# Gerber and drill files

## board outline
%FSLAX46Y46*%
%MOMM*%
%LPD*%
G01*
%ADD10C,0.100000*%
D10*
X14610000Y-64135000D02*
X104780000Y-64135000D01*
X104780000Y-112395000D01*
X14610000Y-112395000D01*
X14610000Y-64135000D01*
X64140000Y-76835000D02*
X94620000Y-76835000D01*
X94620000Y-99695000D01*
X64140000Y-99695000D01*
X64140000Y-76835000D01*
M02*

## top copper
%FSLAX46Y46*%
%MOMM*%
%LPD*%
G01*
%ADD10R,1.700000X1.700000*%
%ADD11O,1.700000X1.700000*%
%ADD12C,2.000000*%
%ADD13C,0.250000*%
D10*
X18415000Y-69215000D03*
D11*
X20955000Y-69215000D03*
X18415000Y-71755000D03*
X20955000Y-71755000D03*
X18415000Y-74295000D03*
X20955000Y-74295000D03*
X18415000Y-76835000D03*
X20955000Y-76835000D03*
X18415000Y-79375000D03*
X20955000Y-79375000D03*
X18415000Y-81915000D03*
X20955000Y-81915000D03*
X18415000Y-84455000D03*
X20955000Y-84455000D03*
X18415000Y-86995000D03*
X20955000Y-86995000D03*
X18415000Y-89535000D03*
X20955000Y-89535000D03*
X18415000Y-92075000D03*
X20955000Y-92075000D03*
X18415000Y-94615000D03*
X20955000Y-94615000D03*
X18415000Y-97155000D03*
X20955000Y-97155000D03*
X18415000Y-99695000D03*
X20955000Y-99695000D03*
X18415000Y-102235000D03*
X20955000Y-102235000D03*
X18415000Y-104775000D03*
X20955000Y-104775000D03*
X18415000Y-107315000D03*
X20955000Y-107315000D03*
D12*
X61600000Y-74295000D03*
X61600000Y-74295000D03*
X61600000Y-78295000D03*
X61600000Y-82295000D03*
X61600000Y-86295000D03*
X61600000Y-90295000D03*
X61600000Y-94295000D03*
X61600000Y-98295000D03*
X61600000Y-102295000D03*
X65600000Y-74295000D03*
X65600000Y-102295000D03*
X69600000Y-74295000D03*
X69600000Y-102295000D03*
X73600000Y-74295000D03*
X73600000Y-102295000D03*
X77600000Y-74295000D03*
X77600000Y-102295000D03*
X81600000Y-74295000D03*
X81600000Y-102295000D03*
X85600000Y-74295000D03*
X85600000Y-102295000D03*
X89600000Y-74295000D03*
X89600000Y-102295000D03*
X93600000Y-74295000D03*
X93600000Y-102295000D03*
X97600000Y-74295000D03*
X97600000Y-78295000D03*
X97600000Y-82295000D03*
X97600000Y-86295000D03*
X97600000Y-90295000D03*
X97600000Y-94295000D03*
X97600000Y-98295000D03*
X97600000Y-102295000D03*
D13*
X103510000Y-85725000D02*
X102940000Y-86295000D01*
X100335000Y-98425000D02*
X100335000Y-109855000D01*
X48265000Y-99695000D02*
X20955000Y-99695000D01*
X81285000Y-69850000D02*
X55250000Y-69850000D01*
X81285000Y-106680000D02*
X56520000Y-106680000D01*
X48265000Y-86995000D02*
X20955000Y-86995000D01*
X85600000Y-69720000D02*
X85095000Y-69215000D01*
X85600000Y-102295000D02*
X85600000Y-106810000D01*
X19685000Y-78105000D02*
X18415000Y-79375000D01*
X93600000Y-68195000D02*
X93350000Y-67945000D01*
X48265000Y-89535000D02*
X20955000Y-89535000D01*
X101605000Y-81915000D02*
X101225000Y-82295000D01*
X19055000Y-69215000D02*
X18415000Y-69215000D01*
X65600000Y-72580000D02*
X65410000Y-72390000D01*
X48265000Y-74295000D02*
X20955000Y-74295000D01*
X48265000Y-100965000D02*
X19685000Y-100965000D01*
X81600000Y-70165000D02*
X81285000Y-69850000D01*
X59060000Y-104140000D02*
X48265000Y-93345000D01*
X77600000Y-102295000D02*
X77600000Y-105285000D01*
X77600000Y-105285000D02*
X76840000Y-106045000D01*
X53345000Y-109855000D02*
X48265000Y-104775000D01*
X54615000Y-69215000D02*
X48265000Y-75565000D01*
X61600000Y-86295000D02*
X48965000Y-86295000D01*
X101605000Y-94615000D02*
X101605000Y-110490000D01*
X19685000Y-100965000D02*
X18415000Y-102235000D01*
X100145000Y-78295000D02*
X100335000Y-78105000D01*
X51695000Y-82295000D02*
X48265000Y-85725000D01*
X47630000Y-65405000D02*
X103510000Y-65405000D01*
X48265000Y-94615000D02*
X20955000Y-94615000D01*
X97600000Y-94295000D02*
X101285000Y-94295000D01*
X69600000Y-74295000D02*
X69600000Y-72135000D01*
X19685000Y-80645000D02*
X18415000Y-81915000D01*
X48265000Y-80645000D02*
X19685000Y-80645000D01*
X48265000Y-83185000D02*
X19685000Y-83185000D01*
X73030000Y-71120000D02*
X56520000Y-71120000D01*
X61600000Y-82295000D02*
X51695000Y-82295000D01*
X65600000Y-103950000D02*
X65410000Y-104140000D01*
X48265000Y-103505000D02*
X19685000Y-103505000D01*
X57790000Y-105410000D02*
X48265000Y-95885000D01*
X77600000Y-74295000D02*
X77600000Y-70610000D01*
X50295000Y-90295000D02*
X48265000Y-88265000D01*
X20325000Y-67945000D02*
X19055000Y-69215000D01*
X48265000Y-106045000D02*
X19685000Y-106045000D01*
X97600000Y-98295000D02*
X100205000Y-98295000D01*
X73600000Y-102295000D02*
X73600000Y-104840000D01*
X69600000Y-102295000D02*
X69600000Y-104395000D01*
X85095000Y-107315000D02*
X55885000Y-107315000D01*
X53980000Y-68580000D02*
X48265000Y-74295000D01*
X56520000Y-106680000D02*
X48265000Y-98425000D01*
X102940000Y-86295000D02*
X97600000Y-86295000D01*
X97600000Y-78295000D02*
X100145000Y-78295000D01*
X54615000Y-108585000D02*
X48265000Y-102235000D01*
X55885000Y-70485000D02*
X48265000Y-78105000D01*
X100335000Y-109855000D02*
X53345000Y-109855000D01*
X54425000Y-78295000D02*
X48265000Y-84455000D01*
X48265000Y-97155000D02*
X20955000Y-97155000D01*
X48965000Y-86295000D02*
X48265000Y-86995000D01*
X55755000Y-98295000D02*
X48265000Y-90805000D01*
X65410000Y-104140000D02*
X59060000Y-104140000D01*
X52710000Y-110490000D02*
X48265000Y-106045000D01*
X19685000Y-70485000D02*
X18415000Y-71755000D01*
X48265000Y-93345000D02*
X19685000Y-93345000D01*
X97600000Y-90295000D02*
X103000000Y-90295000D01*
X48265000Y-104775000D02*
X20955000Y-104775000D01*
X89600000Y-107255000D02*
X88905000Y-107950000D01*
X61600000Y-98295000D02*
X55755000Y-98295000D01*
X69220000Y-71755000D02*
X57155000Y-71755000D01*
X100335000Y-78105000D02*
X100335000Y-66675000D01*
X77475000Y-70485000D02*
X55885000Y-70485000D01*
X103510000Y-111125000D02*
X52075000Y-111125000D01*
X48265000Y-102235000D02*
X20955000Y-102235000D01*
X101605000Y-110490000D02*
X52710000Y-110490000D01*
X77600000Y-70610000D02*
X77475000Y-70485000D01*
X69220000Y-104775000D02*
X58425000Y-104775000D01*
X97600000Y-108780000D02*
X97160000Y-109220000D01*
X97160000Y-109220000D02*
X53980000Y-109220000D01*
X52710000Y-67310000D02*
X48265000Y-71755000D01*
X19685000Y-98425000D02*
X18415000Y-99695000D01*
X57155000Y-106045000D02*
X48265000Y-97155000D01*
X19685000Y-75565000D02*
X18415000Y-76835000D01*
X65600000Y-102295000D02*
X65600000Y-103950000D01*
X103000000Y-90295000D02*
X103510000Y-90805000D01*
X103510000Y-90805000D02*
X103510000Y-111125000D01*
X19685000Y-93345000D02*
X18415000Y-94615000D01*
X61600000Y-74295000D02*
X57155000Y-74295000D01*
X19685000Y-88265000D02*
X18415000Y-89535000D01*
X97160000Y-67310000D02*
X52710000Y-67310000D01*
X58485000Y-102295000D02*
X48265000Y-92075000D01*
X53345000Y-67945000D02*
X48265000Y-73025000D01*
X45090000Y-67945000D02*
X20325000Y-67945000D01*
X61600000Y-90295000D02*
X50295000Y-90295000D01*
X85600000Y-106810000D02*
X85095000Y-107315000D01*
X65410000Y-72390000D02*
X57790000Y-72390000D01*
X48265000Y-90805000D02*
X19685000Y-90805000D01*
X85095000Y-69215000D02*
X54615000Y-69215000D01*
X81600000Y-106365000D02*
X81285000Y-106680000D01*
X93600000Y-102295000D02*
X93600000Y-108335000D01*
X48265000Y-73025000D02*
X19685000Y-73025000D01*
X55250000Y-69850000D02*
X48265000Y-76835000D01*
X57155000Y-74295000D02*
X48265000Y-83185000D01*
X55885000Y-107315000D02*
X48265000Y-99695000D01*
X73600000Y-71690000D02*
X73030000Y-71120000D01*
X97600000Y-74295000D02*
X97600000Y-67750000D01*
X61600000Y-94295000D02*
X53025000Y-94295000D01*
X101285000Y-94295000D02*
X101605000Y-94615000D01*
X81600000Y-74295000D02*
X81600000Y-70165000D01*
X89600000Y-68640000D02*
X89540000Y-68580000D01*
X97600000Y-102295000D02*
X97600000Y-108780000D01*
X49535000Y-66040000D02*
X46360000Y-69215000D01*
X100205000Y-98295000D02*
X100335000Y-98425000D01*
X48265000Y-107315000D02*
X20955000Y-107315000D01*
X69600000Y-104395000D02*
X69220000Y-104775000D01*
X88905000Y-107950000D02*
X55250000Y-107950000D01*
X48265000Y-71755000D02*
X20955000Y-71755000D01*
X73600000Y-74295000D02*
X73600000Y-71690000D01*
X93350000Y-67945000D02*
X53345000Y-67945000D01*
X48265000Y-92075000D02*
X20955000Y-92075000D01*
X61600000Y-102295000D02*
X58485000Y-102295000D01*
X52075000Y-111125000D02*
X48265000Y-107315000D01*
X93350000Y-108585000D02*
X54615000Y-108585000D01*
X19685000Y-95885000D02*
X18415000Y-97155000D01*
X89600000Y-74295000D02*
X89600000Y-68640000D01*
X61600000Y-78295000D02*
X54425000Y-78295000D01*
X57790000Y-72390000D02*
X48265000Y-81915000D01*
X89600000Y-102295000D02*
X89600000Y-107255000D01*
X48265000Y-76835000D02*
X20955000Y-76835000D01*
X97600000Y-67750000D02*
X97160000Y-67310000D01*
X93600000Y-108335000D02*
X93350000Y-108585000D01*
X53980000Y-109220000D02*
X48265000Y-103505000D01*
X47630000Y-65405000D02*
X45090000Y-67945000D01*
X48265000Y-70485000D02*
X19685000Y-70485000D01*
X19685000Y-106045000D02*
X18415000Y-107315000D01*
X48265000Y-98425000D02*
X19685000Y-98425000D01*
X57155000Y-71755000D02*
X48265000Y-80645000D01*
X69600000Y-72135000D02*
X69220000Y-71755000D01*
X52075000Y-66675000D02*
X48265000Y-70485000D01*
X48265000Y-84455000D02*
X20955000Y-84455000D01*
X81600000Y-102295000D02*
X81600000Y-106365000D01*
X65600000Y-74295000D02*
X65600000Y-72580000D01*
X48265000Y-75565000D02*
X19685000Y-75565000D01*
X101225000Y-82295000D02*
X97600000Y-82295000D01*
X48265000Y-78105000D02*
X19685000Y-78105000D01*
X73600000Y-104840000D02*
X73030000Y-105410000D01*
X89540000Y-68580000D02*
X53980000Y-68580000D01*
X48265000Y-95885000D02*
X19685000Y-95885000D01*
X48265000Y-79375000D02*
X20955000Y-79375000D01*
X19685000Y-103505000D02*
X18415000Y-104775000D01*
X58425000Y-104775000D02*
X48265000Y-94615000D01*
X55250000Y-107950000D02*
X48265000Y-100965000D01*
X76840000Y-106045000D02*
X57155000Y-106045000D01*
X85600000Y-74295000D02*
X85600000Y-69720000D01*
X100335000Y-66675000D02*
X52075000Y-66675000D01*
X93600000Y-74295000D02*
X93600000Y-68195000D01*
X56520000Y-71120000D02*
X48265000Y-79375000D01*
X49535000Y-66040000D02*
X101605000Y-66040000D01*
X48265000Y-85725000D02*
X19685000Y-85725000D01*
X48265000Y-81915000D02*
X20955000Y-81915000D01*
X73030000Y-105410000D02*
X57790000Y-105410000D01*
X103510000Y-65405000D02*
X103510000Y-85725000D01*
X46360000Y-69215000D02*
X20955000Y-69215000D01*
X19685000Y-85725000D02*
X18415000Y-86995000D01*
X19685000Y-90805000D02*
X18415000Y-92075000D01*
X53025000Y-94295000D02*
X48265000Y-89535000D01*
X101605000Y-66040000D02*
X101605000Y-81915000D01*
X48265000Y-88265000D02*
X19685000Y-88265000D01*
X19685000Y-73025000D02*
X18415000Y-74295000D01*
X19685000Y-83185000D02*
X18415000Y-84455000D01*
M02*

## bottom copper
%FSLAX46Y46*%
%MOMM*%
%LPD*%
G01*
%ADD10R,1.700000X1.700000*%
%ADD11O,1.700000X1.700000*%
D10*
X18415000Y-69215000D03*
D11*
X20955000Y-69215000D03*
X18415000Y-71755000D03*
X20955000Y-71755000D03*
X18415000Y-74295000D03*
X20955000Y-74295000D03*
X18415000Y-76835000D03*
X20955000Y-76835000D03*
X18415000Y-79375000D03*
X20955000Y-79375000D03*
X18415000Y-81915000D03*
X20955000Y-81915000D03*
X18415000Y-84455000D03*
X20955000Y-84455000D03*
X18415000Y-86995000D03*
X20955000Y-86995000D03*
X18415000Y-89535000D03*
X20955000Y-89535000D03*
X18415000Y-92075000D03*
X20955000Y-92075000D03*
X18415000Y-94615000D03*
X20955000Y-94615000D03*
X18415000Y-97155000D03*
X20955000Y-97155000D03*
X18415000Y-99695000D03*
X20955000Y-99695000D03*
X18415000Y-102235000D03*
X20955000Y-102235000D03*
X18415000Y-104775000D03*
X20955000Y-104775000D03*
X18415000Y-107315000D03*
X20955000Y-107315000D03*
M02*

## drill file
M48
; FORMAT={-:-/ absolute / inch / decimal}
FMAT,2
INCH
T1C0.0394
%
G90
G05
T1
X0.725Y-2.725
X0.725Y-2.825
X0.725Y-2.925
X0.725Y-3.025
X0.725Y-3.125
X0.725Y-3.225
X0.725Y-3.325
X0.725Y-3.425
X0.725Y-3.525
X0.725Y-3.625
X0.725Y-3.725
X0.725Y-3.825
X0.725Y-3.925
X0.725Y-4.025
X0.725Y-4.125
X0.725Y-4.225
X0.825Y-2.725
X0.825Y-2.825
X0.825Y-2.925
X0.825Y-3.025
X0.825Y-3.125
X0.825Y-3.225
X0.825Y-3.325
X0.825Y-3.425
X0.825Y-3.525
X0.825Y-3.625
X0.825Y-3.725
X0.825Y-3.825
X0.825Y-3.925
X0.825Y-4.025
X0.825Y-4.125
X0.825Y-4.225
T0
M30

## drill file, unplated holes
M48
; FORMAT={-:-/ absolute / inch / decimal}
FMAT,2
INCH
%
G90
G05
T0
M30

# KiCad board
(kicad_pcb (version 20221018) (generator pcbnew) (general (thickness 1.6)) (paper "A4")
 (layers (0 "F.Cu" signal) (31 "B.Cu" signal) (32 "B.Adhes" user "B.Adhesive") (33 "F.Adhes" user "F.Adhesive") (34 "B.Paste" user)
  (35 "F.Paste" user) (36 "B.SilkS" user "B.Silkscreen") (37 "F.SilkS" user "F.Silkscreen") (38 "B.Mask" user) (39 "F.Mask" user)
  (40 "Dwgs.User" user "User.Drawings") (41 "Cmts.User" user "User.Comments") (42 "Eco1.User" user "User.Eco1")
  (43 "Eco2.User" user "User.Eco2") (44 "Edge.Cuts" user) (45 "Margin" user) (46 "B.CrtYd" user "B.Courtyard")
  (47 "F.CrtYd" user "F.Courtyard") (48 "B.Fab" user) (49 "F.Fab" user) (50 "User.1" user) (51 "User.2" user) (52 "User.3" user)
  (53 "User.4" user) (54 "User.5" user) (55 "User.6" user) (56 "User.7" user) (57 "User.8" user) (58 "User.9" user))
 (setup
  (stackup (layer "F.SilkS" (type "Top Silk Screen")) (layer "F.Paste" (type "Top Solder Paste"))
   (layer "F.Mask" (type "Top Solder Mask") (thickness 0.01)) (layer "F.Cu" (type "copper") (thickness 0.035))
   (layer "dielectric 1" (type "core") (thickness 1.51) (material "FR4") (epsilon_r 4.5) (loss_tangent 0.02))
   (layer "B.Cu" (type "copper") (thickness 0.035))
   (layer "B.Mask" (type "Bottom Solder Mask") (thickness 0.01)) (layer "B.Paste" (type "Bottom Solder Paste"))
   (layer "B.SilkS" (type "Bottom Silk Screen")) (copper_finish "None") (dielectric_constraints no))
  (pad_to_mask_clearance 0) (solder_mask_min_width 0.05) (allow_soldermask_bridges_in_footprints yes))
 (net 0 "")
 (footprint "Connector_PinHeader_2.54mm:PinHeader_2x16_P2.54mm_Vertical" (layer "F.Cu") (at 18.415 69.215)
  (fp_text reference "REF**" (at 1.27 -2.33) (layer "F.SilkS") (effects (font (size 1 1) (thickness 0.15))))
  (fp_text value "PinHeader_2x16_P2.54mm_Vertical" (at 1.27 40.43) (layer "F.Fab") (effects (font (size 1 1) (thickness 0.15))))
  (pad "1" thru_hole rect (at 0 0) (size 1.7 1.7) (drill 1) (layers "*.Cu" "*.Mask"))
  (pad "2" thru_hole oval (at 2.54 0) (size 1.7 1.7) (drill 1) (layers "*.Cu" "*.Mask"))
  (pad "3" thru_hole oval (at 0 2.54) (size 1.7 1.7) (drill 1) (layers "*.Cu" "*.Mask"))
  (pad "4" thru_hole oval (at 2.54 2.54) (size 1.7 1.7) (drill 1) (layers "*.Cu" "*.Mask"))
  (pad "5" thru_hole oval (at 0 5.08) (size 1.7 1.7) (drill 1) (layers "*.Cu" "*.Mask"))
  (pad "6" thru_hole oval (at 2.54 5.08) (size 1.7 1.7) (drill 1) (layers "*.Cu" "*.Mask"))
  (pad "7" thru_hole oval (at 0 7.62) (size 1.7 1.7) (drill 1) (layers "*.Cu" "*.Mask"))
  (pad "8" thru_hole oval (at 2.54 7.62) (size 1.7 1.7) (drill 1) (layers "*.Cu" "*.Mask"))
  (pad "9" thru_hole oval (at 0 10.16) (size 1.7 1.7) (drill 1) (layers "*.Cu" "*.Mask"))
  (pad "10" thru_hole oval (at 2.54 10.16) (size 1.7 1.7) (drill 1) (layers "*.Cu" "*.Mask"))
  (pad "11" thru_hole oval (at 0 12.7) (size 1.7 1.7) (drill 1) (layers "*.Cu" "*.Mask"))
  (pad "12" thru_hole oval (at 2.54 12.7) (size 1.7 1.7) (drill 1) (layers "*.Cu" "*.Mask"))
  (pad "13" thru_hole oval (at 0 15.24) (size 1.7 1.7) (drill 1) (layers "*.Cu" "*.Mask"))
  (pad "14" thru_hole oval (at 2.54 15.24) (size 1.7 1.7) (drill 1) (layers "*.Cu" "*.Mask"))
  (pad "15" thru_hole oval (at 0 17.78) (size 1.7 1.7) (drill 1) (layers "*.Cu" "*.Mask"))
  (pad "16" thru_hole oval (at 2.54 17.78) (size 1.7 1.7) (drill 1) (layers "*.Cu" "*.Mask"))
  (pad "17" thru_hole oval (at 0 20.32) (size 1.7 1.7) (drill 1) (layers "*.Cu" "*.Mask"))
  (pad "18" thru_hole oval (at 2.54 20.32) (size 1.7 1.7) (drill 1) (layers "*.Cu" "*.Mask"))
  (pad "19" thru_hole oval (at 0 22.86) (size 1.7 1.7) (drill 1) (layers "*.Cu" "*.Mask"))
  (pad "20" thru_hole oval (at 2.54 22.86) (size 1.7 1.7) (drill 1) (layers "*.Cu" "*.Mask"))
  (pad "21" thru_hole oval (at 0 25.4) (size 1.7 1.7) (drill 1) (layers "*.Cu" "*.Mask"))
  (pad "22" thru_hole oval (at 2.54 25.4) (size 1.7 1.7) (drill 1) (layers "*.Cu" "*.Mask"))
  (pad "23" thru_hole oval (at 0 27.94) (size 1.7 1.7) (drill 1) (layers "*.Cu" "*.Mask"))
  (pad "24" thru_hole oval (at 2.54 27.94) (size 1.7 1.7) (drill 1) (layers "*.Cu" "*.Mask"))
  (pad "25" thru_hole oval (at 0 30.48) (size 1.7 1.7) (drill 1) (layers "*.Cu" "*.Mask"))
  (pad "26" thru_hole oval (at 2.54 30.48) (size 1.7 1.7) (drill 1) (layers "*.Cu" "*.Mask"))
  (pad "27" thru_hole oval (at 0 33.02) (size 1.7 1.7) (drill 1) (layers "*.Cu" "*.Mask"))
  (pad "28" thru_hole oval (at 2.54 33.02) (size 1.7 1.7) (drill 1) (layers "*.Cu" "*.Mask"))
  (pad "29" thru_hole oval (at 0 35.56) (size 1.7 1.7) (drill 1) (layers "*.Cu" "*.Mask"))
  (pad "30" thru_hole oval (at 2.54 35.56) (size 1.7 1.7) (drill 1) (layers "*.Cu" "*.Mask"))
  (pad "31" thru_hole oval (at 0 38.1) (size 1.7 1.7) (drill 1) (layers "*.Cu" "*.Mask"))
  (pad "32" thru_hole oval (at 2.54 38.1) (size 1.7 1.7) (drill 1) (layers "*.Cu" "*.Mask")))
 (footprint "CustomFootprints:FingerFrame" (layer "F.Cu") (at 61.6 74.295)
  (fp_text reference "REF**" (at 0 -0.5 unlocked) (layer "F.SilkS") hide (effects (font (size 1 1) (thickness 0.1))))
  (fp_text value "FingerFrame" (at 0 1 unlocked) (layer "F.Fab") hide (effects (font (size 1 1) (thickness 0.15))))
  (pad "1" smd circle (at 0 0) (size 2 2) (layers "F.Cu" "F.Paste" "F.Mask"))
  (pad "1" smd circle (at 0 0) (size 2 2) (layers "F.Cu" "F.Paste" "F.Mask"))
  (pad "1" smd circle (at 0 4) (size 2 2) (layers "F.Cu" "F.Paste" "F.Mask"))
  (pad "1" smd circle (at 0 8) (size 2 2) (layers "F.Cu" "F.Paste" "F.Mask"))
  (pad "1" smd circle (at 0 12) (size 2 2) (layers "F.Cu" "F.Paste" "F.Mask"))
  (pad "1" smd circle (at 0 16) (size 2 2) (layers "F.Cu" "F.Paste" "F.Mask"))
  (pad "1" smd circle (at 0 20) (size 2 2) (layers "F.Cu" "F.Paste" "F.Mask"))
  (pad "1" smd circle (at 0 24) (size 2 2) (layers "F.Cu" "F.Paste" "F.Mask"))
  (pad "1" smd circle (at 0 28) (size 2 2) (layers "F.Cu" "F.Paste" "F.Mask"))
  (pad "1" smd circle (at 4 0) (size 2 2) (layers "F.Cu" "F.Paste" "F.Mask"))
  (pad "1" smd circle (at 4 28) (size 2 2) (layers "F.Cu" "F.Paste" "F.Mask"))
  (pad "1" smd circle (at 8 0) (size 2 2) (layers "F.Cu" "F.Paste" "F.Mask"))
  (pad "1" smd circle (at 8 28) (size 2 2) (layers "F.Cu" "F.Paste" "F.Mask"))
  (pad "1" smd circle (at 12 0) (size 2 2) (layers "F.Cu" "F.Paste" "F.Mask"))
  (pad "1" smd circle (at 12 28) (size 2 2) (layers "F.Cu" "F.Paste" "F.Mask"))
  (pad "1" smd circle (at 16 0) (size 2 2) (layers "F.Cu" "F.Paste" "F.Mask"))
  (pad "1" smd circle (at 16 28) (size 2 2) (layers "F.Cu" "F.Paste" "F.Mask"))
  (pad "1" smd circle (at 20 0) (size 2 2) (layers "F.Cu" "F.Paste" "F.Mask"))
  (pad "1" smd circle (at 20 28) (size 2 2) (layers "F.Cu" "F.Paste" "F.Mask"))
  (pad "1" smd circle (at 24 0) (size 2 2) (layers "F.Cu" "F.Paste" "F.Mask"))
  (pad "1" smd circle (at 24 28) (size 2 2) (layers "F.Cu" "F.Paste" "F.Mask"))
  (pad "1" smd circle (at 28 0) (size 2 2) (layers "F.Cu" "F.Paste" "F.Mask"))
  (pad "1" smd circle (at 28 28) (size 2 2) (layers "F.Cu" "F.Paste" "F.Mask"))
  (pad "1" smd circle (at 32 0) (size 2 2) (layers "F.Cu" "F.Paste" "F.Mask"))
  (pad "1" smd circle (at 32 28) (size 2 2) (layers "F.Cu" "F.Paste" "F.Mask"))
  (pad "1" smd circle (at 36 0) (size 2 2) (layers "F.Cu" "F.Paste" "F.Mask"))
  (pad "1" smd circle (at 36 4) (size 2 2) (layers "F.Cu" "F.Paste" "F.Mask"))
  (pad "1" smd circle (at 36 8) (size 2 2) (layers "F.Cu" "F.Paste" "F.Mask"))
  (pad "1" smd circle (at 36 12) (size 2 2) (layers "F.Cu" "F.Paste" "F.Mask"))
  (pad "1" smd circle (at 36 16) (size 2 2) (layers "F.Cu" "F.Paste" "F.Mask"))
  (pad "1" smd circle (at 36 20) (size 2 2) (layers "F.Cu" "F.Paste" "F.Mask"))
  (pad "1" smd circle (at 36 24) (size 2 2) (layers "F.Cu" "F.Paste" "F.Mask"))
  (pad "1" smd circle (at 36 28) (size 2 2) (layers "F.Cu" "F.Paste" "F.Mask")))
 (gr_rect (start 14.61 64.135) (end 104.78 112.395) (stroke (width 0.1) (type default)) (fill none) (layer "Edge.Cuts"))
 (gr_rect (start 64.14 76.835) (end 94.62 99.695) (stroke (width 0.1) (type default)) (fill none) (layer "Edge.Cuts"))
 (segment (start 103.51 85.725) (end 102.94 86.295) (width 0.25) (layer "F.Cu") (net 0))
 (segment (start 100.335 98.425) (end 100.335 109.855) (width 0.25) (layer "F.Cu") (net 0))
 (segment (start 48.265 99.695) (end 20.955 99.695) (width 0.25) (layer "F.Cu") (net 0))
 (segment (start 81.285 69.85) (end 55.25 69.85) (width 0.25) (layer "F.Cu") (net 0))
 (segment (start 81.285 106.68) (end 56.52 106.68) (width 0.25) (layer "F.Cu") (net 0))
 (segment (start 48.265 86.995) (end 20.955 86.995) (width 0.25) (layer "F.Cu") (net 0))
 (segment (start 85.6 69.72) (end 85.095 69.215) (width 0.25) (layer "F.Cu") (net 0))
 (segment (start 85.6 102.295) (end 85.6 106.81) (width 0.25) (layer "F.Cu") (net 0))
 (segment (start 19.685 78.105) (end 18.415 79.375) (width 0.25) (layer "F.Cu") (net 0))
 (segment (start 93.6 68.195) (end 93.35 67.945) (width 0.25) (layer "F.Cu") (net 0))
 (segment (start 48.265 89.535) (end 20.955 89.535) (width 0.25) (layer "F.Cu") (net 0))
 (segment (start 101.605 81.915) (end 101.225 82.295) (width 0.25) (layer "F.Cu") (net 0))
 (segment (start 19.055 69.215) (end 18.415 69.215) (width 0.25) (layer "F.Cu") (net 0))
 (segment (start 65.6 72.58) (end 65.41 72.39) (width 0.25) (layer "F.Cu") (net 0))
 (segment (start 48.265 74.295) (end 20.955 74.295) (width 0.25) (layer "F.Cu") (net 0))
 (segment (start 48.265 100.965) (end 19.685 100.965) (width 0.25) (layer "F.Cu") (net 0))
 (segment (start 81.6 70.165) (end 81.285 69.85) (width 0.25) (layer "F.Cu") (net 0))
 (segment (start 59.06 104.14) (end 48.265 93.345) (width 0.25) (layer "F.Cu") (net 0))
 (segment (start 77.6 102.295) (end 77.6 105.285) (width 0.25) (layer "F.Cu") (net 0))
 (segment (start 77.6 105.285) (end 76.84 106.045) (width 0.25) (layer "F.Cu") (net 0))
 (segment (start 53.345 109.855) (end 48.265 104.775) (width 0.25) (layer "F.Cu") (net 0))
 (segment (start 54.615 69.215) (end 48.265 75.565) (width 0.25) (layer "F.Cu") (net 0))
 (segment (start 61.6 86.295) (end 48.965 86.295) (width 0.25) (layer "F.Cu") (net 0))
 (segment (start 101.605 94.615) (end 101.605 110.49) (width 0.25) (layer "F.Cu") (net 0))
 (segment (start 19.685 100.965) (end 18.415 102.235) (width 0.25) (layer "F.Cu") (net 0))
 (segment (start 100.145 78.295) (end 100.335 78.105) (width 0.25) (layer "F.Cu") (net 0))
 (segment (start 51.695 82.295) (end 48.265 85.725) (width 0.25) (layer "F.Cu") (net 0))
 (segment (start 47.63 65.405) (end 103.51 65.405) (width 0.25) (layer "F.Cu") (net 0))
 (segment (start 48.265 94.615) (end 20.955 94.615) (width 0.25) (layer "F.Cu") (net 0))
 (segment (start 97.6 94.295) (end 101.285 94.295) (width 0.25) (layer "F.Cu") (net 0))
 (segment (start 69.6 74.295) (end 69.6 72.135) (width 0.25) (layer "F.Cu") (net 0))
 (segment (start 19.685 80.645) (end 18.415 81.915) (width 0.25) (layer "F.Cu") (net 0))
 (segment (start 48.265 80.645) (end 19.685 80.645) (width 0.25) (layer "F.Cu") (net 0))
 (segment (start 48.265 83.185) (end 19.685 83.185) (width 0.25) (layer "F.Cu") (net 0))
 (segment (start 73.03 71.12) (end 56.52 71.12) (width 0.25) (layer "F.Cu") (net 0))
 (segment (start 61.6 82.295) (end 51.695 82.295) (width 0.25) (layer "F.Cu") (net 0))
 (segment (start 65.6 103.95) (end 65.41 104.14) (width 0.25) (layer "F.Cu") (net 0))
 (segment (start 48.265 103.505) (end 19.685 103.505) (width 0.25) (layer "F.Cu") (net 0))
 (segment (start 57.79 105.41) (end 48.265 95.885) (width 0.25) (layer "F.Cu") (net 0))
 (segment (start 77.6 74.295) (end 77.6 70.61) (width 0.25) (layer "F.Cu") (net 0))
 (segment (start 50.295 90.295) (end 48.265 88.265) (width 0.25) (layer "F.Cu") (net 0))
 (segment (start 20.325 67.945) (end 19.055 69.215) (width 0.25) (layer "F.Cu") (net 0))
 (segment (start 48.265 106.045) (end 19.685 106.045) (width 0.25) (layer "F.Cu") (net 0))
 (segment (start 97.6 98.295) (end 100.205 98.295) (width 0.25) (layer "F.Cu") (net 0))
 (segment (start 73.6 102.295) (end 73.6 104.84) (width 0.25) (layer "F.Cu") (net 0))
 (segment (start 69.6 102.295) (end 69.6 104.395) (width 0.25) (layer "F.Cu") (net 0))
 (segment (start 85.095 107.315) (end 55.885 107.315) (width 0.25) (layer "F.Cu") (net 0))
 (segment (start 53.98 68.58) (end 48.265 74.295) (width 0.25) (layer "F.Cu") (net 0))
 (segment (start 56.52 106.68) (end 48.265 98.425) (width 0.25) (layer "F.Cu") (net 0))
 (segment (start 102.94 86.295) (end 97.6 86.295) (width 0.25) (layer "F.Cu") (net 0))
 (segment (start 97.6 78.295) (end 100.145 78.295) (width 0.25) (layer "F.Cu") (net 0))
 (segment (start 54.615 108.585) (end 48.265 102.235) (width 0.25) (layer "F.Cu") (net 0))
 (segment (start 55.885 70.485) (end 48.265 78.105) (width 0.25) (layer "F.Cu") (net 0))
 (segment (start 100.335 109.855) (end 53.345 109.855) (width 0.25) (layer "F.Cu") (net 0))
 (segment (start 54.425 78.295) (end 48.265 84.455) (width 0.25) (layer "F.Cu") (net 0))
 (segment (start 48.265 97.155) (end 20.955 97.155) (width 0.25) (layer "F.Cu") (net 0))
 (segment (start 48.965 86.295) (end 48.265 86.995) (width 0.25) (layer "F.Cu") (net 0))
 (segment (start 55.755 98.295) (end 48.265 90.805) (width 0.25) (layer "F.Cu") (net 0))
 (segment (start 65.41 104.14) (end 59.06 104.14) (width 0.25) (layer "F.Cu") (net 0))
 (segment (start 52.71 110.49) (end 48.265 106.045) (width 0.25) (layer "F.Cu") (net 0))
 (segment (start 19.685 70.485) (end 18.415 71.755) (width 0.25) (layer "F.Cu") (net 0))
 (segment (start 48.265 93.345) (end 19.685 93.345) (width 0.25) (layer "F.Cu") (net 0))
 (segment (start 97.6 90.295) (end 103 90.295) (width 0.25) (layer "F.Cu") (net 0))
 (segment (start 48.265 104.775) (end 20.955 104.775) (width 0.25) (layer "F.Cu") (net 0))
 (segment (start 89.6 107.255) (end 88.905 107.95) (width 0.25) (layer "F.Cu") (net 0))
 (segment (start 61.6 98.295) (end 55.755 98.295) (width 0.25) (layer "F.Cu") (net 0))
 (segment (start 69.22 71.755) (end 57.155 71.755) (width 0.25) (layer "F.Cu") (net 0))
 (segment (start 100.335 78.105) (end 100.335 66.675) (width 0.25) (layer "F.Cu") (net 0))
 (segment (start 77.475 70.485) (end 55.885 70.485) (width 0.25) (layer "F.Cu") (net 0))
 (segment (start 103.51 111.125) (end 52.075 111.125) (width 0.25) (layer "F.Cu") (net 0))
 (segment (start 48.265 102.235) (end 20.955 102.235) (width 0.25) (layer "F.Cu") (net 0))
 (segment (start 101.605 110.49) (end 52.71 110.49) (width 0.25) (layer "F.Cu") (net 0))
 (segment (start 77.6 70.61) (end 77.475 70.485) (width 0.25) (layer "F.Cu") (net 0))
 (segment (start 69.22 104.775) (end 58.425 104.775) (width 0.25) (layer "F.Cu") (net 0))
 (segment (start 97.6 108.78) (end 97.16 109.22) (width 0.25) (layer "F.Cu") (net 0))
 (segment (start 97.16 109.22) (end 53.98 109.22) (width 0.25) (layer "F.Cu") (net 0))
 (segment (start 52.71 67.31) (end 48.265 71.755) (width 0.25) (layer "F.Cu") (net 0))
 (segment (start 19.685 98.425) (end 18.415 99.695) (width 0.25) (layer "F.Cu") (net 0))
 (segment (start 57.155 106.045) (end 48.265 97.155) (width 0.25) (layer "F.Cu") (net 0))
 (segment (start 19.685 75.565) (end 18.415 76.835) (width 0.25) (layer "F.Cu") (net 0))
 (segment (start 65.6 102.295) (end 65.6 103.95) (width 0.25) (layer "F.Cu") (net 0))
 (segment (start 103 90.295) (end 103.51 90.805) (width 0.25) (layer "F.Cu") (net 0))
 (segment (start 103.51 90.805) (end 103.51 111.125) (width 0.25) (layer "F.Cu") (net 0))
 (segment (start 19.685 93.345) (end 18.415 94.615) (width 0.25) (layer "F.Cu") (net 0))
 (segment (start 61.6 74.295) (end 57.155 74.295) (width 0.25) (layer "F.Cu") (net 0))
 (segment (start 19.685 88.265) (end 18.415 89.535) (width 0.25) (layer "F.Cu") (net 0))
 (segment (start 97.16 67.31) (end 52.71 67.31) (width 0.25) (layer "F.Cu") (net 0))
 (segment (start 58.485 102.295) (end 48.265 92.075) (width 0.25) (layer "F.Cu") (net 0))
 (segment (start 53.345 67.945) (end 48.265 73.025) (width 0.25) (layer "F.Cu") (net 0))
 (segment (start 45.09 67.945) (end 20.325 67.945) (width 0.25) (layer "F.Cu") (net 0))
 (segment (start 61.6 90.295) (end 50.295 90.295) (width 0.25) (layer "F.Cu") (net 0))
 (segment (start 85.6 106.81) (end 85.095 107.315) (width 0.25) (layer "F.Cu") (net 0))
 (segment (start 65.41 72.39) (end 57.79 72.39) (width 0.25) (layer "F.Cu") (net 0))
 (segment (start 48.265 90.805) (end 19.685 90.805) (width 0.25) (layer "F.Cu") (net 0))
 (segment (start 85.095 69.215) (end 54.615 69.215) (width 0.25) (layer "F.Cu") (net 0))
 (segment (start 81.6 106.365) (end 81.285 106.68) (width 0.25) (layer "F.Cu") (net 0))
 (segment (start 93.6 102.295) (end 93.6 108.335) (width 0.25) (layer "F.Cu") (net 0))
 (segment (start 48.265 73.025) (end 19.685 73.025) (width 0.25) (layer "F.Cu") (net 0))
 (segment (start 55.25 69.85) (end 48.265 76.835) (width 0.25) (layer "F.Cu") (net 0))
 (segment (start 57.155 74.295) (end 48.265 83.185) (width 0.25) (layer "F.Cu") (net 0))
 (segment (start 55.885 107.315) (end 48.265 99.695) (width 0.25) (layer "F.Cu") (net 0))
 (segment (start 73.6 71.69) (end 73.03 71.12) (width 0.25) (layer "F.Cu") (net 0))
 (segment (start 97.6 74.295) (end 97.6 67.75) (width 0.25) (layer "F.Cu") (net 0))
 (segment (start 61.6 94.295) (end 53.025 94.295) (width 0.25) (layer "F.Cu") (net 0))
 (segment (start 101.285 94.295) (end 101.605 94.615) (width 0.25) (layer "F.Cu") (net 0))
 (segment (start 81.6 74.295) (end 81.6 70.165) (width 0.25) (layer "F.Cu") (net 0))
 (segment (start 89.6 68.64) (end 89.54 68.58) (width 0.25) (layer "F.Cu") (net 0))
 (segment (start 97.6 102.295) (end 97.6 108.78) (width 0.25) (layer "F.Cu") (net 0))
 (segment (start 49.535 66.04) (end 46.36 69.215) (width 0.25) (layer "F.Cu") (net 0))
 (segment (start 100.205 98.295) (end 100.335 98.425) (width 0.25) (layer "F.Cu") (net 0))
 (segment (start 48.265 107.315) (end 20.955 107.315) (width 0.25) (layer "F.Cu") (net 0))
 (segment (start 69.6 104.395) (end 69.22 104.775) (width 0.25) (layer "F.Cu") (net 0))
 (segment (start 88.905 107.95) (end 55.25 107.95) (width 0.25) (layer "F.Cu") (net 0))
 (segment (start 48.265 71.755) (end 20.955 71.755) (width 0.25) (layer "F.Cu") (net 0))
 (segment (start 73.6 74.295) (end 73.6 71.69) (width 0.25) (layer "F.Cu") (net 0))
 (segment (start 93.35 67.945) (end 53.345 67.945) (width 0.25) (layer "F.Cu") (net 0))
 (segment (start 48.265 92.075) (end 20.955 92.075) (width 0.25) (layer "F.Cu") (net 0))
 (segment (start 61.6 102.295) (end 58.485 102.295) (width 0.25) (layer "F.Cu") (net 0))
 (segment (start 52.075 111.125) (end 48.265 107.315) (width 0.25) (layer "F.Cu") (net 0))
 (segment (start 93.35 108.585) (end 54.615 108.585) (width 0.25) (layer "F.Cu") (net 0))
 (segment (start 19.685 95.885) (end 18.415 97.155) (width 0.25) (layer "F.Cu") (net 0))
 (segment (start 89.6 74.295) (end 89.6 68.64) (width 0.25) (layer "F.Cu") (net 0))
 (segment (start 61.6 78.295) (end 54.425 78.295) (width 0.25) (layer "F.Cu") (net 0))
 (segment (start 57.79 72.39) (end 48.265 81.915) (width 0.25) (layer "F.Cu") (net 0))
 (segment (start 89.6 102.295) (end 89.6 107.255) (width 0.25) (layer "F.Cu") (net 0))
 (segment (start 48.265 76.835) (end 20.955 76.835) (width 0.25) (layer "F.Cu") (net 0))
 (segment (start 97.6 67.75) (end 97.16 67.31) (width 0.25) (layer "F.Cu") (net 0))
 (segment (start 93.6 108.335) (end 93.35 108.585) (width 0.25) (layer "F.Cu") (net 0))
 (segment (start 53.98 109.22) (end 48.265 103.505) (width 0.25) (layer "F.Cu") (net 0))
 (segment (start 47.63 65.405) (end 45.09 67.945) (width 0.25) (layer "F.Cu") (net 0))
 (segment (start 48.265 70.485) (end 19.685 70.485) (width 0.25) (layer "F.Cu") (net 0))
 (segment (start 19.685 106.045) (end 18.415 107.315) (width 0.25) (layer "F.Cu") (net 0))
 (segment (start 48.265 98.425) (end 19.685 98.425) (width 0.25) (layer "F.Cu") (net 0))
 (segment (start 57.155 71.755) (end 48.265 80.645) (width 0.25) (layer "F.Cu") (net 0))
 (segment (start 69.6 72.135) (end 69.22 71.755) (width 0.25) (layer "F.Cu") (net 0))
 (segment (start 52.075 66.675) (end 48.265 70.485) (width 0.25) (layer "F.Cu") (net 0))
 (segment (start 48.265 84.455) (end 20.955 84.455) (width 0.25) (layer "F.Cu") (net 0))
 (segment (start 81.6 102.295) (end 81.6 106.365) (width 0.25) (layer "F.Cu") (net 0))
 (segment (start 65.6 74.295) (end 65.6 72.58) (width 0.25) (layer "F.Cu") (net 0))
 (segment (start 48.265 75.565) (end 19.685 75.565) (width 0.25) (layer "F.Cu") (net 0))
 (segment (start 101.225 82.295) (end 97.6 82.295) (width 0.25) (layer "F.Cu") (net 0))
 (segment (start 48.265 78.105) (end 19.685 78.105) (width 0.25) (layer "F.Cu") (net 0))
 (segment (start 73.6 104.84) (end 73.03 105.41) (width 0.25) (layer "F.Cu") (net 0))
 (segment (start 89.54 68.58) (end 53.98 68.58) (width 0.25) (layer "F.Cu") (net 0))
 (segment (start 48.265 95.885) (end 19.685 95.885) (width 0.25) (layer "F.Cu") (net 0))
 (segment (start 48.265 79.375) (end 20.955 79.375) (width 0.25) (layer "F.Cu") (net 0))
 (segment (start 19.685 103.505) (end 18.415 104.775) (width 0.25) (layer "F.Cu") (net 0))
 (segment (start 58.425 104.775) (end 48.265 94.615) (width 0.25) (layer "F.Cu") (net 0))
 (segment (start 55.25 107.95) (end 48.265 100.965) (width 0.25) (layer "F.Cu") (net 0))
 (segment (start 76.84 106.045) (end 57.155 106.045) (width 0.25) (layer "F.Cu") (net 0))
 (segment (start 85.6 74.295) (end 85.6 69.72) (width 0.25) (layer "F.Cu") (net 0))
 (segment (start 100.335 66.675) (end 52.075 66.675) (width 0.25) (layer "F.Cu") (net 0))
 (segment (start 93.6 74.295) (end 93.6 68.195) (width 0.25) (layer "F.Cu") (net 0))
 (segment (start 56.52 71.12) (end 48.265 79.375) (width 0.25) (layer "F.Cu") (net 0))
 (segment (start 49.535 66.04) (end 101.605 66.04) (width 0.25) (layer "F.Cu") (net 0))
 (segment (start 48.265 85.725) (end 19.685 85.725) (width 0.25) (layer "F.Cu") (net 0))
 (segment (start 48.265 81.915) (end 20.955 81.915) (width 0.25) (layer "F.Cu") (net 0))
 (segment (start 73.03 105.41) (end 57.79 105.41) (width 0.25) (layer "F.Cu") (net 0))
 (segment (start 103.51 65.405) (end 103.51 85.725) (width 0.25) (layer "F.Cu") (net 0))
 (segment (start 46.36 69.215) (end 20.955 69.215) (width 0.25) (layer "F.Cu") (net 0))
 (segment (start 19.685 85.725) (end 18.415 86.995) (width 0.25) (layer "F.Cu") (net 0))
 (segment (start 19.685 90.805) (end 18.415 92.075) (width 0.25) (layer "F.Cu") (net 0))
 (segment (start 53.025 94.295) (end 48.265 89.535) (width 0.25) (layer "F.Cu") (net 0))
 (segment (start 101.605 66.04) (end 101.605 81.915) (width 0.25) (layer "F.Cu") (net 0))
 (segment (start 48.265 88.265) (end 19.685 88.265) (width 0.25) (layer "F.Cu") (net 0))
 (segment (start 19.685 73.025) (end 18.415 74.295) (width 0.25) (layer "F.Cu") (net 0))
 (segment (start 19.685 83.185) (end 18.415 84.455) (width 0.25) (layer "F.Cu") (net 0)))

